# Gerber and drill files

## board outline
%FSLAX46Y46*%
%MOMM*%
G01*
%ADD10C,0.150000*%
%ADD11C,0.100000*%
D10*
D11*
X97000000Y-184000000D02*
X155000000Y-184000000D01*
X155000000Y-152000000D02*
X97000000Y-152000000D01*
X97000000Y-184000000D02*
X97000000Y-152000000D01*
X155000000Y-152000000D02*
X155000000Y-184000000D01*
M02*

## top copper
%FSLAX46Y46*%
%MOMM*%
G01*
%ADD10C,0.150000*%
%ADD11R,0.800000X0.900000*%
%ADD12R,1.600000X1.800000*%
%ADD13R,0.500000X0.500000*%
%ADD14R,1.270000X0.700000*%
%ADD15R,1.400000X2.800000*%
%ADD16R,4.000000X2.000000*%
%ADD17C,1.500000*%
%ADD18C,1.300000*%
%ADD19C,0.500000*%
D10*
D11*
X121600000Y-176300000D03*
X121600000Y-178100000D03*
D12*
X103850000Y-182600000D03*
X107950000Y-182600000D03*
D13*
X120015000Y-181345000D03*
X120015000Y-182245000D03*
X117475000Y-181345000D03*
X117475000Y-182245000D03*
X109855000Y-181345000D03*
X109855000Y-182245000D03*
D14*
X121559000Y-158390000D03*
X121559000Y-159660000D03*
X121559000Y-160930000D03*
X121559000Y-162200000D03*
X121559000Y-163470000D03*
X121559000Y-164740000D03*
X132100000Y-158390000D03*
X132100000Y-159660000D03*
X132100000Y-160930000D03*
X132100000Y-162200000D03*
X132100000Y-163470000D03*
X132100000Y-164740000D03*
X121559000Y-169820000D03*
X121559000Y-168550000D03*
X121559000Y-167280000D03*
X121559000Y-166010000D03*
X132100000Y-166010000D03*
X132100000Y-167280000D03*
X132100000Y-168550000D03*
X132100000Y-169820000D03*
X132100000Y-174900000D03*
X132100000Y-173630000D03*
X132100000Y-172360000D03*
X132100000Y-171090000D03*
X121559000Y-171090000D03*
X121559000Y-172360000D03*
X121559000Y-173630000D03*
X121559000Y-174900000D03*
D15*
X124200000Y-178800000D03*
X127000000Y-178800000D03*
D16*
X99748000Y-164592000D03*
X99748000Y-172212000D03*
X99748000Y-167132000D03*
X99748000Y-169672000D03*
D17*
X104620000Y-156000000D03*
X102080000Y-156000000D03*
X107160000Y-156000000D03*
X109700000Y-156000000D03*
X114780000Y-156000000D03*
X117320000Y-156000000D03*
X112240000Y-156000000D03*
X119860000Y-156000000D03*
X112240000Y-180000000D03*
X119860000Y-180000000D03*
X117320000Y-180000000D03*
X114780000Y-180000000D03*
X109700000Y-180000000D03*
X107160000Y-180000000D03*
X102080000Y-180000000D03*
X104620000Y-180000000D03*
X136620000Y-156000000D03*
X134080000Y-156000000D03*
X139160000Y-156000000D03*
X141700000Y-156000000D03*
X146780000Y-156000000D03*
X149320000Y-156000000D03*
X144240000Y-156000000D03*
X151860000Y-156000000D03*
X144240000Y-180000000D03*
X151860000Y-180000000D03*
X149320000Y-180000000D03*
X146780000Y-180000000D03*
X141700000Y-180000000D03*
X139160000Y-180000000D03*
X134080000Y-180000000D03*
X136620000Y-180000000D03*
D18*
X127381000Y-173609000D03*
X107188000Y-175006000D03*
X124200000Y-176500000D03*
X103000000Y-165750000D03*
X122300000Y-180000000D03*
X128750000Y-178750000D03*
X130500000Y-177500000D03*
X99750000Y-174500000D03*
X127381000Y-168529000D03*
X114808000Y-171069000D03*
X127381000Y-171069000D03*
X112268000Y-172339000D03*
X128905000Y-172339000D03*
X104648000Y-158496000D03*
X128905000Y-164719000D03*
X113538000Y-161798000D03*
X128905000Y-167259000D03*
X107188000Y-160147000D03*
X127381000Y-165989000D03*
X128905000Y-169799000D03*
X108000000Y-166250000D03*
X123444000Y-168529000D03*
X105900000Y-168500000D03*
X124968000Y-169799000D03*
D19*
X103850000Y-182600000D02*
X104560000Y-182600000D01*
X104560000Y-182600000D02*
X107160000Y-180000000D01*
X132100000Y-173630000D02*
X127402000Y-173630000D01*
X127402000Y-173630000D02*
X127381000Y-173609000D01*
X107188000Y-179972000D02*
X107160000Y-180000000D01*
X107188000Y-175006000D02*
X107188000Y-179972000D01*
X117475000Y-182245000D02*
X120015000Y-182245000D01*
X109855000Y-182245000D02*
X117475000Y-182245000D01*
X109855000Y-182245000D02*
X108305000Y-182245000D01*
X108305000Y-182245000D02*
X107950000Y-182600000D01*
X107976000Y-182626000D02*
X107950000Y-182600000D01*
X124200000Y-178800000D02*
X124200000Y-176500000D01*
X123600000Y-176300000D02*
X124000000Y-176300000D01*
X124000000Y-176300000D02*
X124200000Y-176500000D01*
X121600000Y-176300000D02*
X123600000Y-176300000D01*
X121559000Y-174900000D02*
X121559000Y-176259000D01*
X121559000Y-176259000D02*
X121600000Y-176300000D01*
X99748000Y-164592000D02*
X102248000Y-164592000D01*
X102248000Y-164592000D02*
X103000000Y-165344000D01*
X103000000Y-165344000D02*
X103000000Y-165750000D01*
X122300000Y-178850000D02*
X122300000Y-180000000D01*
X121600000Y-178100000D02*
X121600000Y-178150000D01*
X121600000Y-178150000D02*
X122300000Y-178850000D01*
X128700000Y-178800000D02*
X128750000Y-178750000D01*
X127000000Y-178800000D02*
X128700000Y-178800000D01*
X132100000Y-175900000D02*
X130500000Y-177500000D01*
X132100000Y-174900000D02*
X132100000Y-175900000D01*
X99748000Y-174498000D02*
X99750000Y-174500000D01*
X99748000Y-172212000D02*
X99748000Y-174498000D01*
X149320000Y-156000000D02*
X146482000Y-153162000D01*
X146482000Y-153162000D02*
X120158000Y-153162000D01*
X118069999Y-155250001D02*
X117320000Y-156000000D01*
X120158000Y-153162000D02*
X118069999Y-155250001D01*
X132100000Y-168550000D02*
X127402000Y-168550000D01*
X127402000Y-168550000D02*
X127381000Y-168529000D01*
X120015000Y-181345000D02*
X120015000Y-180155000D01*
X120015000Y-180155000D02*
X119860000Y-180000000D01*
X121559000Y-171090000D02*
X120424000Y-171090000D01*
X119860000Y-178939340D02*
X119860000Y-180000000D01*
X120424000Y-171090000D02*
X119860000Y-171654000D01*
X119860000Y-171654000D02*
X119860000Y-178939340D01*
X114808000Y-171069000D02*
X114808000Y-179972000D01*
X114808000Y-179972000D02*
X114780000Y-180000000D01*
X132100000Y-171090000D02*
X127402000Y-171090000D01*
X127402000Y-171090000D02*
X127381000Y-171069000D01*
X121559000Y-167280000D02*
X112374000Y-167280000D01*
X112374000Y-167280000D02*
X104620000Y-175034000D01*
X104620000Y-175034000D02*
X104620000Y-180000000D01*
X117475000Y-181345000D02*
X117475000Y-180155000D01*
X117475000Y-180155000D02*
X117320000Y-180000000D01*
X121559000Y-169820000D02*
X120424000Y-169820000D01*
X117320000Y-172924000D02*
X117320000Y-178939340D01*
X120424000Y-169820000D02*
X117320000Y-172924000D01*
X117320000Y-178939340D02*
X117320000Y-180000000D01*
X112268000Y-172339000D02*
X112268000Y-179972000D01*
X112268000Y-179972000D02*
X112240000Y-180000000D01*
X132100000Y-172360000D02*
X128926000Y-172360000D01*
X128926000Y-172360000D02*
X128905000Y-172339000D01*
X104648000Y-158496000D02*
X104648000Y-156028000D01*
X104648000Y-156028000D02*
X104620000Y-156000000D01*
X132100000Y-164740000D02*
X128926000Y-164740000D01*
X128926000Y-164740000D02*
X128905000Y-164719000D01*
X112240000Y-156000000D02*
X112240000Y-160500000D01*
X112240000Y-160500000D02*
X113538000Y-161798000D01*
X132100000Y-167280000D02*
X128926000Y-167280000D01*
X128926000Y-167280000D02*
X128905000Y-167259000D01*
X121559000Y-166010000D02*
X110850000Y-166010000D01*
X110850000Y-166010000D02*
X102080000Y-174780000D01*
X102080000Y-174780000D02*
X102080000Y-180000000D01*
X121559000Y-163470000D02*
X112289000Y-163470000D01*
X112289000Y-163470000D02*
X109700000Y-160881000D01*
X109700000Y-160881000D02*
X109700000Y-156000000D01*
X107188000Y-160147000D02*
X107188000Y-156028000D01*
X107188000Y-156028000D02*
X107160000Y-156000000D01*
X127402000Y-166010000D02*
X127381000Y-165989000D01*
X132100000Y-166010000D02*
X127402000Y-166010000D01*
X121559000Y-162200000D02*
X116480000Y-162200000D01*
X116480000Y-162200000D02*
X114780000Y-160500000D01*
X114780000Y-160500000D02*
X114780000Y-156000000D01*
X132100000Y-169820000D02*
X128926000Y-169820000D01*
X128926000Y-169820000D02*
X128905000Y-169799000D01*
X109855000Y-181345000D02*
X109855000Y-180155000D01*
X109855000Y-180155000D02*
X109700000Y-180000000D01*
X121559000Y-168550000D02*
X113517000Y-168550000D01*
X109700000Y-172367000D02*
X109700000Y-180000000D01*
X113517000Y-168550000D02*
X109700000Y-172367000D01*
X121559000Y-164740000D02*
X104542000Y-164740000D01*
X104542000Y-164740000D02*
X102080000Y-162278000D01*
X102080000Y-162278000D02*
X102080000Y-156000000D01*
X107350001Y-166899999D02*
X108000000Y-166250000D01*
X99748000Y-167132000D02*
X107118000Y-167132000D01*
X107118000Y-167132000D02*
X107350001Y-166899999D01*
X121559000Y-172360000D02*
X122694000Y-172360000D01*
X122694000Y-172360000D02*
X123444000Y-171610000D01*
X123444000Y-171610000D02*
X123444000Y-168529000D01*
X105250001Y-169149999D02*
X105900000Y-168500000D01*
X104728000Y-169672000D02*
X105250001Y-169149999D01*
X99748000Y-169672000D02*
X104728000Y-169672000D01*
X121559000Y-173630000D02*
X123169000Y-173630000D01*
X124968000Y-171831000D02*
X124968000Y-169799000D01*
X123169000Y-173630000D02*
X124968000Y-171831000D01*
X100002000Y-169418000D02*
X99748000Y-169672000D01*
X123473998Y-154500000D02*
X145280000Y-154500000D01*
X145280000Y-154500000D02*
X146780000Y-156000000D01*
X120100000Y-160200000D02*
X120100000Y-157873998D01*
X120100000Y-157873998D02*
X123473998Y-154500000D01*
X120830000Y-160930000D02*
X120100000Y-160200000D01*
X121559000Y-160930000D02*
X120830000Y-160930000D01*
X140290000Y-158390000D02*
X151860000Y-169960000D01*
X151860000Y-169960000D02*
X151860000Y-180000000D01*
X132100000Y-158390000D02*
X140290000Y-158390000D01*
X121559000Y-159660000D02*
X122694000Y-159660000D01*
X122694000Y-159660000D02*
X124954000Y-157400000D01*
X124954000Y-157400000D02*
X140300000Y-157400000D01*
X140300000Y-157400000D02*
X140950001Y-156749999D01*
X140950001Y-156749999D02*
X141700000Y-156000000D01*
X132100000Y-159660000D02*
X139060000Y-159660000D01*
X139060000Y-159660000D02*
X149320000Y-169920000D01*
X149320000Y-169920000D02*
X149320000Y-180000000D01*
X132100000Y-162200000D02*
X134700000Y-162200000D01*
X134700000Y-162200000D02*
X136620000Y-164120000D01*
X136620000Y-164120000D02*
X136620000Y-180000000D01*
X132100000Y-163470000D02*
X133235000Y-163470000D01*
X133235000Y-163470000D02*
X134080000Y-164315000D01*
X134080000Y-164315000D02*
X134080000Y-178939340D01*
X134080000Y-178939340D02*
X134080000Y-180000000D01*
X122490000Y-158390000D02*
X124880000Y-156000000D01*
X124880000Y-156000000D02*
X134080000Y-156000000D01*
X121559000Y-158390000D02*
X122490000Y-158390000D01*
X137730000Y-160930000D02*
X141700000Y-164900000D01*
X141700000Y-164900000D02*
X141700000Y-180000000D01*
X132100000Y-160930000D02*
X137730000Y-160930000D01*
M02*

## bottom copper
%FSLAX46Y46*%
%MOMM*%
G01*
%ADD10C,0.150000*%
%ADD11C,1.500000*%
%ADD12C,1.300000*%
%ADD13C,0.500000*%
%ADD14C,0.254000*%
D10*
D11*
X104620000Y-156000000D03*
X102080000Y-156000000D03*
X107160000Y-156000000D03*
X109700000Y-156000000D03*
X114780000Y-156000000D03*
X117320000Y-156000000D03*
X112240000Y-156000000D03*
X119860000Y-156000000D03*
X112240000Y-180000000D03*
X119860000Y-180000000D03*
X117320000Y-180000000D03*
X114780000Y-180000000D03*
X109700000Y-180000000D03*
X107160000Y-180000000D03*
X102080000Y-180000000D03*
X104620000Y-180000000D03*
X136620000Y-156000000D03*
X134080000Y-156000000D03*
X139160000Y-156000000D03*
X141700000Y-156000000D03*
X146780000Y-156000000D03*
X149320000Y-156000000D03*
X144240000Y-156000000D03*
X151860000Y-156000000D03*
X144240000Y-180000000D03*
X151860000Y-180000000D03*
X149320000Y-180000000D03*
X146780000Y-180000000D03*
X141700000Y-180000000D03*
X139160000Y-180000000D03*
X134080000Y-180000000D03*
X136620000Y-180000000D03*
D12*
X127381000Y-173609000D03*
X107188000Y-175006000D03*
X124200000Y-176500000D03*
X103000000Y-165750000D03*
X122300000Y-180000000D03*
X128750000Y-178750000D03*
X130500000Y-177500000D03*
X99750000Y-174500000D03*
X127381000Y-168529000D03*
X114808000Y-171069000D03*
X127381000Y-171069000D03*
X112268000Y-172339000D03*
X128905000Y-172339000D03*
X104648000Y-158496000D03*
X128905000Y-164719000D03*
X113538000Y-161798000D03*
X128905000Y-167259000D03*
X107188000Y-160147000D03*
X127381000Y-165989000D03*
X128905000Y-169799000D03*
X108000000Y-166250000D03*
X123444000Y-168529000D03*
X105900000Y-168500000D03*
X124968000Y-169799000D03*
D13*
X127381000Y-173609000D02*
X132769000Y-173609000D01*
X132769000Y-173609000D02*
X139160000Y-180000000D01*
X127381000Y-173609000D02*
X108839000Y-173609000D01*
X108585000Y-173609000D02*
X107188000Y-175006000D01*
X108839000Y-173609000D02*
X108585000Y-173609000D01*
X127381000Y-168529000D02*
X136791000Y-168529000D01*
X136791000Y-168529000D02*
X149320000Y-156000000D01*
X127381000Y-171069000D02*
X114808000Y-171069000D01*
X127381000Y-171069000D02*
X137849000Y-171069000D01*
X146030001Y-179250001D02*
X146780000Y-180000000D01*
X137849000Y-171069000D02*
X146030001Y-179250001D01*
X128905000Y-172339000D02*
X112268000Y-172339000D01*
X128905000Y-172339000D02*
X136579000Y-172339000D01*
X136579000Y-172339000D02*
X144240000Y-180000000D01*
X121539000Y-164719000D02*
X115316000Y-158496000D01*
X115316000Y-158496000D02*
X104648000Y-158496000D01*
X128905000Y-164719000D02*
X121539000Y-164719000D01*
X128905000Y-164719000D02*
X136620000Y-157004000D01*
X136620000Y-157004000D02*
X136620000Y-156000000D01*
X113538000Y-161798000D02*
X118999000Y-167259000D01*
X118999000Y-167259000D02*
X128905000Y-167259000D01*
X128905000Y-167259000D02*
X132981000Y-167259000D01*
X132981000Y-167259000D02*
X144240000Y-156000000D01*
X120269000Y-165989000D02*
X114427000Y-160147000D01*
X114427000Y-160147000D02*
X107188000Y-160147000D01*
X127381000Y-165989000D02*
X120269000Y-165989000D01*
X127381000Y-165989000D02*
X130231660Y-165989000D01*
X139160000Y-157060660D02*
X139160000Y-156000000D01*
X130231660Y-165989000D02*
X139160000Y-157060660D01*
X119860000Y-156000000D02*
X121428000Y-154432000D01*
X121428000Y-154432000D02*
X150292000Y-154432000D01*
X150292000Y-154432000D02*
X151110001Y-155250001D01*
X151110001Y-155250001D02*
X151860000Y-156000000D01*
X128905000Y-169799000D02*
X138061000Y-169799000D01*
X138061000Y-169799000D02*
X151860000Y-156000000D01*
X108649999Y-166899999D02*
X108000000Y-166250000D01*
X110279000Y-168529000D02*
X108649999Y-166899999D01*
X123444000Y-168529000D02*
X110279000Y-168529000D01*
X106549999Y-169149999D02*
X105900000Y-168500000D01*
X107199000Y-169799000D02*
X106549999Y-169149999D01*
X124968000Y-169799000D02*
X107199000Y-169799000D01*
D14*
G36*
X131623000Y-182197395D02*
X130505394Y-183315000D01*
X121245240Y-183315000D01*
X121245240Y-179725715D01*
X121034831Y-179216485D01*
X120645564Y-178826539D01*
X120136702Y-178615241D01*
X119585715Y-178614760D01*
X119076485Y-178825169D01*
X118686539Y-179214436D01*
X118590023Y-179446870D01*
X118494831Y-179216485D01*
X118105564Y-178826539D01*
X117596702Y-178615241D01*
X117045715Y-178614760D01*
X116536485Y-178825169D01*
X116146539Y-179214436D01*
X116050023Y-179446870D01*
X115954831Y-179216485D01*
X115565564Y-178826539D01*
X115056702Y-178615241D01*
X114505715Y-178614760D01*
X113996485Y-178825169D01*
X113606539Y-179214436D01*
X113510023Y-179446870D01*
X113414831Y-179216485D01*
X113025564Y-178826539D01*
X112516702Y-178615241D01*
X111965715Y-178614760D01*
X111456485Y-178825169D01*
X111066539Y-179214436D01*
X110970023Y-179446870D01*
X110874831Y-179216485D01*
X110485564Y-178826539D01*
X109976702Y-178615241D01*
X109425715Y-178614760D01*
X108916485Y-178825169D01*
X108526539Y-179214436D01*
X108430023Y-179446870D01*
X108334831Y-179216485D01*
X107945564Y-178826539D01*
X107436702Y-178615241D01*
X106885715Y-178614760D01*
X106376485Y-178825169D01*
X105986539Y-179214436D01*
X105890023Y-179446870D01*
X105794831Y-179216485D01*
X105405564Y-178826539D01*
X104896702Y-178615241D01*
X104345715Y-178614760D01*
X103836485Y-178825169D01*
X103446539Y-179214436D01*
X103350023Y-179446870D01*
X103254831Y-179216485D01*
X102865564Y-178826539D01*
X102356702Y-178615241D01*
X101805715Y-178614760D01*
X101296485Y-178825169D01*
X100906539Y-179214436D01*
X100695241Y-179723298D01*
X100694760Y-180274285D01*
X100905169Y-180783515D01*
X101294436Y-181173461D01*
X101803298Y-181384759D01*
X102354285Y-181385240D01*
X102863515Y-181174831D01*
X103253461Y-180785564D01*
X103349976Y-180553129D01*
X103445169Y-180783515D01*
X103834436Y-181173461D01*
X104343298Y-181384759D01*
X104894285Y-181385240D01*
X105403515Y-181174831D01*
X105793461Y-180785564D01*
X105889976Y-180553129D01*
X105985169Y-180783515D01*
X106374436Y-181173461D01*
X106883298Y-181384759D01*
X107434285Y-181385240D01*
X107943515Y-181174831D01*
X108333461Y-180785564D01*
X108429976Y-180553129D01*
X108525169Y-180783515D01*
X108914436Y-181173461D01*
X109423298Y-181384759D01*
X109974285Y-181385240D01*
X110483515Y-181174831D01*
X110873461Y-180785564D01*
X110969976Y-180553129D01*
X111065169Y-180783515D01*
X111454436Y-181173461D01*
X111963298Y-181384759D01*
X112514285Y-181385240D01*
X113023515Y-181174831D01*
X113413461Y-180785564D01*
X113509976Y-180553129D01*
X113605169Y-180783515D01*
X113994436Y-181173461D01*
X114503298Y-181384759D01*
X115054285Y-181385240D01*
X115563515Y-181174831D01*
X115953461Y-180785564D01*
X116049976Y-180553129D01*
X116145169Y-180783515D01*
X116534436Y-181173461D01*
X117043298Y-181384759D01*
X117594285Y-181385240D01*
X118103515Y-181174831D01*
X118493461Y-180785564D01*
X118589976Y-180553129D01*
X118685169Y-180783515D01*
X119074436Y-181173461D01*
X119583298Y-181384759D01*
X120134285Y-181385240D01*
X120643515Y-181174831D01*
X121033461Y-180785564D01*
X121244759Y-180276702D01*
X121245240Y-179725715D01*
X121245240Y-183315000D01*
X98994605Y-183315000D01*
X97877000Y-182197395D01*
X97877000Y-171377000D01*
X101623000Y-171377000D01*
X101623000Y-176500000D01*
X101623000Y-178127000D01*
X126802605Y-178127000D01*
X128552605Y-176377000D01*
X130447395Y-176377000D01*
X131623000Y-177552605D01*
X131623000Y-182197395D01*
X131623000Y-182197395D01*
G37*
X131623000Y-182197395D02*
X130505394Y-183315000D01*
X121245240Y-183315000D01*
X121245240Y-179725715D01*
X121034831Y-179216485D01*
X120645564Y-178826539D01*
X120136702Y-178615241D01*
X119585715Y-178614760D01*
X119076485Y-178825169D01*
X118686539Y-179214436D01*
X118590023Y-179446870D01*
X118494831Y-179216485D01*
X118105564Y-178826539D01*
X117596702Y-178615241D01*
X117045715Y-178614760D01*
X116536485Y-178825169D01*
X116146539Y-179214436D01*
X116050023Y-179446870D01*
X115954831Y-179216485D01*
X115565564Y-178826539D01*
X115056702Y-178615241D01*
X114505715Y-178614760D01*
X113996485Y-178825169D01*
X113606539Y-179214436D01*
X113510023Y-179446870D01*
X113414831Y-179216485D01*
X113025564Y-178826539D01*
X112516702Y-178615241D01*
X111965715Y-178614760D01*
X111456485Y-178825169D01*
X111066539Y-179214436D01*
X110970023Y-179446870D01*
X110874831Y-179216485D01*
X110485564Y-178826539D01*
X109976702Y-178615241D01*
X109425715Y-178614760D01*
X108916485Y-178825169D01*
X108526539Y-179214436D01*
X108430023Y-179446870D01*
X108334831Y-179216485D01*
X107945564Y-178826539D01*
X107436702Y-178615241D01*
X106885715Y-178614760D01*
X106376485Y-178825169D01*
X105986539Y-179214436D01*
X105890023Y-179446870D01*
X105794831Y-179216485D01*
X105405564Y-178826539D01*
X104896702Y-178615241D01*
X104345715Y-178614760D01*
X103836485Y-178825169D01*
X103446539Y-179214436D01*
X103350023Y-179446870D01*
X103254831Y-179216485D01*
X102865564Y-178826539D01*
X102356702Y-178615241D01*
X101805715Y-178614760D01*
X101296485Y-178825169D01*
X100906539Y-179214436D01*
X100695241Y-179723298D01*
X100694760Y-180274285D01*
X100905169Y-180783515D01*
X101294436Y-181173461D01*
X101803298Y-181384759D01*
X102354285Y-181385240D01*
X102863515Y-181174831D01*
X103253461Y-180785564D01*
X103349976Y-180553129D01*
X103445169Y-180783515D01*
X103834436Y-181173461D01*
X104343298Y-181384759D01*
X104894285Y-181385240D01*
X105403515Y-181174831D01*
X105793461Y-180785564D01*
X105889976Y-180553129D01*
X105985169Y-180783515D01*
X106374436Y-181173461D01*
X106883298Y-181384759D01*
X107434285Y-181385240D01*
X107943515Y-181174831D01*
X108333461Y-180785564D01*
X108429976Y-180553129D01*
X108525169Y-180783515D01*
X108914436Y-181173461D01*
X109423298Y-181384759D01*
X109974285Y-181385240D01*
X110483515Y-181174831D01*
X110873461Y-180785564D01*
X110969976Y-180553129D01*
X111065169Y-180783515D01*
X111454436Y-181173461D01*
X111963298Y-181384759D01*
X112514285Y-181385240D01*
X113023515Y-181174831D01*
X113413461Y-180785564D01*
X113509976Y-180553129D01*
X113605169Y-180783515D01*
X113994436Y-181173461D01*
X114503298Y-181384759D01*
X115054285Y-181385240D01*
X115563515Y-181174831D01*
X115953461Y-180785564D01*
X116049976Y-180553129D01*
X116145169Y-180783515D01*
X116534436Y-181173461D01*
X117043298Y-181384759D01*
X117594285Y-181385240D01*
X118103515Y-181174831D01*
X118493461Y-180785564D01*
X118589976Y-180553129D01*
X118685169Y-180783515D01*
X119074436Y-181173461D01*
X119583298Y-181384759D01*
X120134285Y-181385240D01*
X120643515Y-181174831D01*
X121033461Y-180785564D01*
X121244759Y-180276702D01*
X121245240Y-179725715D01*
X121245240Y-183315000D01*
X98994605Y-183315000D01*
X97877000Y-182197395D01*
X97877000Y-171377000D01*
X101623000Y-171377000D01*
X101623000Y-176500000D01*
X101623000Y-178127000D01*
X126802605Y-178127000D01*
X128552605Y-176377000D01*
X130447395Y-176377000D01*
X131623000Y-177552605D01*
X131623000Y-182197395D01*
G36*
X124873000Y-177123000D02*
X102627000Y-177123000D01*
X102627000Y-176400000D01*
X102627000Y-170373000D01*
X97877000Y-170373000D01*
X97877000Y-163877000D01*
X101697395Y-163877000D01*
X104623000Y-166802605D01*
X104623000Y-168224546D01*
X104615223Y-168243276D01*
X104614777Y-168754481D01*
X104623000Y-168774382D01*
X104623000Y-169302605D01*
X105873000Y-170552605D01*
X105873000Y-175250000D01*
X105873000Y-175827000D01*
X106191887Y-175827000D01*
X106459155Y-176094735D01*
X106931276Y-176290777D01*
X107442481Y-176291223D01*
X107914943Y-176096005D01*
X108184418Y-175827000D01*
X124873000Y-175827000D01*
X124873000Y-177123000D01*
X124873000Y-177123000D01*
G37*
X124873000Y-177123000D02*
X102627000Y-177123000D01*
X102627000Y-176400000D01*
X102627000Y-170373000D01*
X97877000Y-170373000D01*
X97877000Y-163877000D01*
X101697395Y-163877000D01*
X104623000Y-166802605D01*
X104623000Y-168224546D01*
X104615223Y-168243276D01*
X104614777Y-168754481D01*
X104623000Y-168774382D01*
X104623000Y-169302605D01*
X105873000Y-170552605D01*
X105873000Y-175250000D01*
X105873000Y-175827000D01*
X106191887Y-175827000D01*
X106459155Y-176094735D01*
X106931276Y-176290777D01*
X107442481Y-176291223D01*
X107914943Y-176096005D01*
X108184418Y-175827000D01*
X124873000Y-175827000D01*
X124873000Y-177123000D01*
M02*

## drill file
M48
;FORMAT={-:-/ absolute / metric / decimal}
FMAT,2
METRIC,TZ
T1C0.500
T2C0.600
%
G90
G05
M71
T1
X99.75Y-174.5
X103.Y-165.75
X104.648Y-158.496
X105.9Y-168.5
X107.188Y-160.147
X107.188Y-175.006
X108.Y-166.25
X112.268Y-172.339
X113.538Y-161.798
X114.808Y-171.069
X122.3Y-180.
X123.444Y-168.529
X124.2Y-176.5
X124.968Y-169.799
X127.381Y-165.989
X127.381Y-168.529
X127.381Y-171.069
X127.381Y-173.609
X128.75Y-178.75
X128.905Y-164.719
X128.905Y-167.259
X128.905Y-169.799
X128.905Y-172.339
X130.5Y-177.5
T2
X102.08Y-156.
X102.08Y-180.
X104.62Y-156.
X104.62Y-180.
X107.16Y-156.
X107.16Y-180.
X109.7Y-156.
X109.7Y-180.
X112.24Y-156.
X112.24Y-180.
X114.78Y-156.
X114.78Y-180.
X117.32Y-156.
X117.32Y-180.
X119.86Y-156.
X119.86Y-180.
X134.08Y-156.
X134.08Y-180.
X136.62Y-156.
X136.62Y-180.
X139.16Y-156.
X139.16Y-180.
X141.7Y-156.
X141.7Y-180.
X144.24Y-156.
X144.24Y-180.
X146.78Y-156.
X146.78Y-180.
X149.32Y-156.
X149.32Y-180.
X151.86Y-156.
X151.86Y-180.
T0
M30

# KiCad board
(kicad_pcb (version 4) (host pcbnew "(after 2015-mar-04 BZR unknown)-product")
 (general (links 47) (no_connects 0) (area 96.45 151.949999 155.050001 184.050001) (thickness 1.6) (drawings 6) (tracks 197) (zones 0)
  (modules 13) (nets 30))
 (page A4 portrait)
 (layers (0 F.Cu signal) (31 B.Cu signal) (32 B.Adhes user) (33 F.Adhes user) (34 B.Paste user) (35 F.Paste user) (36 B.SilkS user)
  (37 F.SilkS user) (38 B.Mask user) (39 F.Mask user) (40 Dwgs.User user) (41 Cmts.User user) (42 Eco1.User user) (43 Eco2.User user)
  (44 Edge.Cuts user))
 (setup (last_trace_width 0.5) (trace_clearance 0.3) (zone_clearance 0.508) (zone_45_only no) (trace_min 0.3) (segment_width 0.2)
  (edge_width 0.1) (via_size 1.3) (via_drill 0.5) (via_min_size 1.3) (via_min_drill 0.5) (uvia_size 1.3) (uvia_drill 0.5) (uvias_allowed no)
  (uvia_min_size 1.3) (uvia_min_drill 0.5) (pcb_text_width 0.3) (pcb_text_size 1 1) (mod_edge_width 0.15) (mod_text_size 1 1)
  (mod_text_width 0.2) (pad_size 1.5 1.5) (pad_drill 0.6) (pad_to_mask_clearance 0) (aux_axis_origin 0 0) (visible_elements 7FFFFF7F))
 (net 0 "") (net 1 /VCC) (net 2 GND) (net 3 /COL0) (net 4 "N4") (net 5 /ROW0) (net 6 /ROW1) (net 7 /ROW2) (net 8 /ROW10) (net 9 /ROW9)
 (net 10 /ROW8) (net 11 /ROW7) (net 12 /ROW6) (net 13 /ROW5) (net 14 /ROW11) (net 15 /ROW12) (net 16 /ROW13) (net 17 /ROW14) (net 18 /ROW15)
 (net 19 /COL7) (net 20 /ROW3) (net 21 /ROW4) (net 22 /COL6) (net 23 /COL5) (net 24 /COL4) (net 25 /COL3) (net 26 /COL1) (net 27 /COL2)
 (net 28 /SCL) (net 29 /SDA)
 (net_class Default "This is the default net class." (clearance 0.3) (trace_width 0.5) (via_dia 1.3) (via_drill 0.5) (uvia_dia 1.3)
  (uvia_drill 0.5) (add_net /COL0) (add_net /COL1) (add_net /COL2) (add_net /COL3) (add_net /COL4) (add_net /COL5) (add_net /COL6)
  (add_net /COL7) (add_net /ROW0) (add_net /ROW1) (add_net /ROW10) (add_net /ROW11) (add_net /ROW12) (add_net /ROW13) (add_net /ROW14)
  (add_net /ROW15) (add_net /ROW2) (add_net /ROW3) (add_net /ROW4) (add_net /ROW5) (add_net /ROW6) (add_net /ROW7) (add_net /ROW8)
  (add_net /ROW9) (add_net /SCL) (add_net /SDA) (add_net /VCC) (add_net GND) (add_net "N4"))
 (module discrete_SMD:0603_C (layer F.Cu) (at 121.6 176.45 270)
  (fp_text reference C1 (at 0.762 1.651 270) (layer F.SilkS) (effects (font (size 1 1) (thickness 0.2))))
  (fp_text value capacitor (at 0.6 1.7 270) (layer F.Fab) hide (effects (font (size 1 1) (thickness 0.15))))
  (pad 1 smd rect (at -0.15 0 270) (size 0.9 0.8) (layers F.Cu F.Paste F.Mask) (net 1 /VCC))
  (pad 2 smd rect (at 1.65 0 270) (size 0.9 0.8) (layers F.Cu F.Paste F.Mask) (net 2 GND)))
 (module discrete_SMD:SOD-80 (layer F.Cu) (at 104.25 182.6 270)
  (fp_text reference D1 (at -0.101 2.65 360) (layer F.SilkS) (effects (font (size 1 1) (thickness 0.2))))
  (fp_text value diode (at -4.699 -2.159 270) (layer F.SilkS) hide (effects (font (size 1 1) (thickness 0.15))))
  (pad 1 smd rect (at 0 0.4 270) (size 1.8 1.6) (layers F.Cu F.Paste F.Mask) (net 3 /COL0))
  (pad 2 smd rect (at 0 -3.7 270) (size 1.8 1.6) (layers F.Cu F.Paste F.Mask) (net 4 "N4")))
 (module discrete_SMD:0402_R (layer F.Cu) (at 120.015 181.345 270)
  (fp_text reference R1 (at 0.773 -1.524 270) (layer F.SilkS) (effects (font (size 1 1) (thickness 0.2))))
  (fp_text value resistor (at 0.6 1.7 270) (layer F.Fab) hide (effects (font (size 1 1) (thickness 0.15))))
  (pad 1 smd rect (at 0 0 270) (size 0.5 0.5) (layers F.Cu F.Paste F.Mask) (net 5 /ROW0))
  (pad 2 smd rect (at 0.9 0 270) (size 0.5 0.5) (layers F.Cu F.Paste F.Mask) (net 4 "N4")))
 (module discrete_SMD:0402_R (layer F.Cu) (at 117.475 181.345 270)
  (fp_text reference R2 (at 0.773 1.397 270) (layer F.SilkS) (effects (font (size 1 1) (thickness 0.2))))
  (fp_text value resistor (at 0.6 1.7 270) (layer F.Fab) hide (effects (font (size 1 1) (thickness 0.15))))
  (pad 1 smd rect (at 0 0 270) (size 0.5 0.5) (layers F.Cu F.Paste F.Mask) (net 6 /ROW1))
  (pad 2 smd rect (at 0.9 0 270) (size 0.5 0.5) (layers F.Cu F.Paste F.Mask) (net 4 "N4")))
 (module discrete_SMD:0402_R (layer F.Cu) (at 109.855 181.345 270)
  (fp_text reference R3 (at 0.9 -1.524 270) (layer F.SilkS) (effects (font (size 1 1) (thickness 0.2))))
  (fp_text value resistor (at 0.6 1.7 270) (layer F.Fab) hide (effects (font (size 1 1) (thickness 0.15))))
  (pad 1 smd rect (at 0 0 270) (size 0.5 0.5) (layers F.Cu F.Paste F.Mask) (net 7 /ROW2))
  (pad 2 smd rect (at 0.9 0 270) (size 0.5 0.5) (layers F.Cu F.Paste F.Mask) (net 4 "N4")))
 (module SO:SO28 (layer F.Cu) (at 132.1 174.9 90)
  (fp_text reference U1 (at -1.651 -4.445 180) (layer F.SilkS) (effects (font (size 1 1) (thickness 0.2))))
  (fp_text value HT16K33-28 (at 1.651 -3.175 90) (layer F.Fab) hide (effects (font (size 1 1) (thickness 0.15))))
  (pad 15 smd rect (at 16.51 -10.541 90) (size 0.7 1.27) (layers F.Cu F.Paste F.Mask) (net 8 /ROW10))
  (pad 16 smd rect (at 15.24 -10.541 90) (size 0.7 1.27) (layers F.Cu F.Paste F.Mask) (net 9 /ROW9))
  (pad 17 smd rect (at 13.97 -10.541 90) (size 0.7 1.27) (layers F.Cu F.Paste F.Mask) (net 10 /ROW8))
  (pad 18 smd rect (at 12.7 -10.541 90) (size 0.7 1.27) (layers F.Cu F.Paste F.Mask) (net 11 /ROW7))
  (pad 19 smd rect (at 11.43 -10.541 90) (size 0.7 1.27) (layers F.Cu F.Paste F.Mask) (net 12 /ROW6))
  (pad 20 smd rect (at 10.16 -10.541 90) (size 0.7 1.27) (layers F.Cu F.Paste F.Mask) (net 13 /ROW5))
  (pad 14 smd rect (at 16.51 0 90) (size 0.7 1.27) (layers F.Cu F.Paste F.Mask) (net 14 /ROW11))
  (pad 13 smd rect (at 15.24 0 90) (size 0.7 1.27) (layers F.Cu F.Paste F.Mask) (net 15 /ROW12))
  (pad 12 smd rect (at 13.97 0 90) (size 0.7 1.27) (layers F.Cu F.Paste F.Mask) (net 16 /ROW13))
  (pad 11 smd rect (at 12.7 0 90) (size 0.7 1.27) (layers F.Cu F.Paste F.Mask) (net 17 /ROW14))
  (pad 10 smd rect (at 11.43 0 90) (size 0.7 1.27) (layers F.Cu F.Paste F.Mask) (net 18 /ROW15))
  (pad 9 smd rect (at 10.16 0 90) (size 0.7 1.27) (layers F.Cu F.Paste F.Mask) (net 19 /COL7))
  (pad 24 smd rect (at 5.08 -10.541 90) (size 0.7 1.27) (layers F.Cu F.Paste F.Mask) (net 6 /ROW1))
  (pad 23 smd rect (at 6.35 -10.541 90) (size 0.7 1.27) (layers F.Cu F.Paste F.Mask) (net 7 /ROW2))
  (pad 22 smd rect (at 7.62 -10.541 90) (size 0.7 1.27) (layers F.Cu F.Paste F.Mask) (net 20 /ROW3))
  (pad 21 smd rect (at 8.89 -10.541 90) (size 0.7 1.27) (layers F.Cu F.Paste F.Mask) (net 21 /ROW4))
  (pad 8 smd rect (at 8.89 0 90) (size 0.7 1.27) (layers F.Cu F.Paste F.Mask) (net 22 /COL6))
  (pad 7 smd rect (at 7.62 0 90) (size 0.7 1.27) (layers F.Cu F.Paste F.Mask) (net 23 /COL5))
  (pad 6 smd rect (at 6.35 0 90) (size 0.7 1.27) (layers F.Cu F.Paste F.Mask) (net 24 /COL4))
  (pad 5 smd rect (at 5.08 0 90) (size 0.7 1.27) (layers F.Cu F.Paste F.Mask) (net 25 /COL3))
  (pad 1 smd rect (at 0 0 90) (size 0.7 1.27) (layers F.Cu F.Paste F.Mask) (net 2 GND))
  (pad 2 smd rect (at 1.27 0 90) (size 0.7 1.27) (layers F.Cu F.Paste F.Mask) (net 3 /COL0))
  (pad 3 smd rect (at 2.54 0 90) (size 0.7 1.27) (layers F.Cu F.Paste F.Mask) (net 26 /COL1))
  (pad 4 smd rect (at 3.81 0 90) (size 0.7 1.27) (layers F.Cu F.Paste F.Mask) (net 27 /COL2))
  (pad 25 smd rect (at 3.81 -10.541 90) (size 0.7 1.27) (layers F.Cu F.Paste F.Mask) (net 5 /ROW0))
  (pad 26 smd rect (at 2.54 -10.541 90) (size 0.7 1.27) (layers F.Cu F.Paste F.Mask) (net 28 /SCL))
  (pad 27 smd rect (at 1.27 -10.541 90) (size 0.7 1.27) (layers F.Cu F.Paste F.Mask) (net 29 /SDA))
  (pad 28 smd rect (at 0 -10.541 90) (size 0.7 1.27) (layers F.Cu F.Paste F.Mask) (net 1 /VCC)))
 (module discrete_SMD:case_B (layer F.Cu) (at 125.65 178.8)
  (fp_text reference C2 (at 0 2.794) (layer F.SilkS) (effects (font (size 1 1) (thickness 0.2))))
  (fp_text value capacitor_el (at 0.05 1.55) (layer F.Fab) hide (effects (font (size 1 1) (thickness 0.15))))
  (pad 1 smd rect (at -1.45 0) (size 1.4 2.8) (layers F.Cu F.Paste F.Mask) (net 1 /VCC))
  (pad 2 smd rect (at 1.35 0) (size 1.4 2.8) (layers F.Cu F.Paste F.Mask) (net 2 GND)))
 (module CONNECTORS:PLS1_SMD (layer F.Cu) (at 98.298 164.592)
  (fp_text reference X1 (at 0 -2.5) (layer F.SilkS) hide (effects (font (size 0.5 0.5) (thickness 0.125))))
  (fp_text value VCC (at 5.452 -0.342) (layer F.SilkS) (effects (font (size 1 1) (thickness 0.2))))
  (pad 1 smd rect (at 1.45 0) (size 4 2) (layers F.Cu F.Paste F.Mask) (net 1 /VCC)))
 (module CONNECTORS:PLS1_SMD (layer F.Cu) (at 98.298 172.212)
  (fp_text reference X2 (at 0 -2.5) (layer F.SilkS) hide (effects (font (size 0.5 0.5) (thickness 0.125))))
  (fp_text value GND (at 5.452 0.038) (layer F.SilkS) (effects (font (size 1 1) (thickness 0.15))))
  (pad 1 smd rect (at 1.45 0) (size 4 2) (layers F.Cu F.Paste F.Mask) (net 2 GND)))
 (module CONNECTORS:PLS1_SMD (layer F.Cu) (at 98.298 167.132)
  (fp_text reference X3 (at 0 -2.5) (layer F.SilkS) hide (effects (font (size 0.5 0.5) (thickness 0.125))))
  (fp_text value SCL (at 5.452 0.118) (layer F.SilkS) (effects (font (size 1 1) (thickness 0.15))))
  (pad 1 smd rect (at 1.45 0) (size 4 2) (layers F.Cu F.Paste F.Mask) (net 28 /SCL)))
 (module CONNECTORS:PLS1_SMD (layer F.Cu) (at 98.298 169.672)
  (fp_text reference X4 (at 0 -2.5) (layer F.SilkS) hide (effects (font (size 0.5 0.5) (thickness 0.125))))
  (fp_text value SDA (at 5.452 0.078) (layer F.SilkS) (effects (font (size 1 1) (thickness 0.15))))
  (pad 1 smd rect (at 1.45 0) (size 4 2) (layers F.Cu F.Paste F.Mask) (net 29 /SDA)))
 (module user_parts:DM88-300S (layer B.Cu) (at 97 156)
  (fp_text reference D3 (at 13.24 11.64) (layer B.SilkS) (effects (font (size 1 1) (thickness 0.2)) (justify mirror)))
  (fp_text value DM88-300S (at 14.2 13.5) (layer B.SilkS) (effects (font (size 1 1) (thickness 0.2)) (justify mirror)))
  (pad 2 thru_hole circle (at 7.62 0) (size 1.5 1.5) (drill 0.6) (layers *.Cu *.Mask) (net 19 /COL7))
  (pad 1 thru_hole circle (at 5.08 0) (size 1.5 1.5) (drill 0.6) (layers *.Cu *.Mask) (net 13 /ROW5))
  (pad 3 thru_hole circle (at 10.16 0) (size 1.5 1.5) (drill 0.6) (layers *.Cu *.Mask) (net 22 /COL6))
  (pad 4 thru_hole circle (at 12.7 0) (size 1.5 1.5) (drill 0.6) (layers *.Cu *.Mask) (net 12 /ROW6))
  (pad 6 thru_hole circle (at 17.78 0) (size 1.5 1.5) (drill 0.6) (layers *.Cu *.Mask) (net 11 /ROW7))
  (pad 7 thru_hole circle (at 20.32 0) (size 1.5 1.5) (drill 0.6) (layers *.Cu *.Mask) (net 24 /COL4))
  (pad 5 thru_hole circle (at 15.24 0) (size 1.5 1.5) (drill 0.6) (layers *.Cu *.Mask) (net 23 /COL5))
  (pad 8 thru_hole circle (at 22.86 0) (size 1.5 1.5) (drill 0.6) (layers *.Cu *.Mask) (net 25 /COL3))
  (pad 12 thru_hole circle (at 15.24 24) (size 1.5 1.5) (drill 0.6) (layers *.Cu *.Mask) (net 26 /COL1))
  (pad 9 thru_hole circle (at 22.86 24) (size 1.5 1.5) (drill 0.6) (layers *.Cu *.Mask) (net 5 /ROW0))
  (pad 10 thru_hole circle (at 20.32 24) (size 1.5 1.5) (drill 0.6) (layers *.Cu *.Mask) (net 6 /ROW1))
  (pad 11 thru_hole circle (at 17.78 24) (size 1.5 1.5) (drill 0.6) (layers *.Cu *.Mask) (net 27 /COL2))
  (pad 13 thru_hole circle (at 12.7 24) (size 1.5 1.5) (drill 0.6) (layers *.Cu *.Mask) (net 7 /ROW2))
  (pad 14 thru_hole circle (at 10.16 24) (size 1.5 1.5) (drill 0.6) (layers *.Cu *.Mask) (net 3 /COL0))
  (pad 16 thru_hole circle (at 5.08 24) (size 1.5 1.5) (drill 0.6) (layers *.Cu *.Mask) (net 21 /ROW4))
  (pad 15 thru_hole circle (at 7.62 24) (size 1.5 1.5) (drill 0.6) (layers *.Cu *.Mask) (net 20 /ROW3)))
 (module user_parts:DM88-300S (layer B.Cu) (at 129 156)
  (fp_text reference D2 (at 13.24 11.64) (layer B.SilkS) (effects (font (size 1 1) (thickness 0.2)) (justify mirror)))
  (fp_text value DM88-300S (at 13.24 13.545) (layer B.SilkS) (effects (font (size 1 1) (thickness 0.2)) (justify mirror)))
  (pad 2 thru_hole circle (at 7.62 0) (size 1.5 1.5) (drill 0.6) (layers *.Cu *.Mask) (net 19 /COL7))
  (pad 1 thru_hole circle (at 5.08 0) (size 1.5 1.5) (drill 0.6) (layers *.Cu *.Mask) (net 8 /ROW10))
  (pad 3 thru_hole circle (at 10.16 0) (size 1.5 1.5) (drill 0.6) (layers *.Cu *.Mask) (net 22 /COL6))
  (pad 4 thru_hole circle (at 12.7 0) (size 1.5 1.5) (drill 0.6) (layers *.Cu *.Mask) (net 9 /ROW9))
  (pad 6 thru_hole circle (at 17.78 0) (size 1.5 1.5) (drill 0.6) (layers *.Cu *.Mask) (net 10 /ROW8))
  (pad 7 thru_hole circle (at 20.32 0) (size 1.5 1.5) (drill 0.6) (layers *.Cu *.Mask) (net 24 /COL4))
  (pad 5 thru_hole circle (at 15.24 0) (size 1.5 1.5) (drill 0.6) (layers *.Cu *.Mask) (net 23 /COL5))
  (pad 8 thru_hole circle (at 22.86 0) (size 1.5 1.5) (drill 0.6) (layers *.Cu *.Mask) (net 25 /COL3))
  (pad 12 thru_hole circle (at 15.24 24) (size 1.5 1.5) (drill 0.6) (layers *.Cu *.Mask) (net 26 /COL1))
  (pad 9 thru_hole circle (at 22.86 24) (size 1.5 1.5) (drill 0.6) (layers *.Cu *.Mask) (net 14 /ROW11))
  (pad 10 thru_hole circle (at 20.32 24) (size 1.5 1.5) (drill 0.6) (layers *.Cu *.Mask) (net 15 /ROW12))
  (pad 11 thru_hole circle (at 17.78 24) (size 1.5 1.5) (drill 0.6) (layers *.Cu *.Mask) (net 27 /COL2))
  (pad 13 thru_hole circle (at 12.7 24) (size 1.5 1.5) (drill 0.6) (layers *.Cu *.Mask) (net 16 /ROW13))
  (pad 14 thru_hole circle (at 10.16 24) (size 1.5 1.5) (drill 0.6) (layers *.Cu *.Mask) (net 3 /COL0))
  (pad 16 thru_hole circle (at 5.08 24) (size 1.5 1.5) (drill 0.6) (layers *.Cu *.Mask) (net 18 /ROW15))
  (pad 15 thru_hole circle (at 7.62 24) (size 1.5 1.5) (drill 0.6) (layers *.Cu *.Mask) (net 17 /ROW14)))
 (gr_line (start 97 184) (end 155 184) (angle 90) (layer Edge.Cuts) (width 0.1))
 (gr_line (start 155 152) (end 97 152) (angle 90) (layer Edge.Cuts) (width 0.1))
 (gr_line (start 97 184) (end 97 152) (angle 90) (layer Edge.Cuts) (width 0.1))
 (gr_line (start 155 152) (end 155 184) (angle 90) (layer Edge.Cuts) (width 0.1))
 (segment (start 103.85 182.6) (end 104.56 182.6) (width 0.5) (layer F.Cu) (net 3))
 (segment (start 104.56 182.6) (end 107.16 180) (width 0.5) (layer F.Cu) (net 3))
 (segment (start 127.381 173.609) (end 132.769 173.609) (width 0.5) (layer B.Cu) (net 3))
 (segment (start 132.769 173.609) (end 139.16 180) (width 0.5) (layer B.Cu) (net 3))
 (segment (start 132.1 173.63) (end 127.402 173.63) (width 0.5) (layer F.Cu) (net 3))
 (via (at 127.381 173.609) (size 1.3) (drill 0.5) (layers F.Cu B.Cu) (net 3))
 (segment (start 127.402 173.63) (end 127.381 173.609) (width 0.5) (layer F.Cu) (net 3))
 (segment (start 127.381 173.609) (end 108.839 173.609) (width 0.5) (layer B.Cu) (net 3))
 (via (at 107.188 175.006) (size 1.3) (drill 0.5) (layers F.Cu B.Cu) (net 3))
 (segment (start 108.585 173.609) (end 107.188 175.006) (width 0.5) (layer B.Cu) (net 3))
 (segment (start 108.839 173.609) (end 108.585 173.609) (width 0.5) (layer B.Cu) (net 3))
 (segment (start 107.188 179.972) (end 107.16 180) (width 0.5) (layer F.Cu) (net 3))
 (segment (start 107.188 175.006) (end 107.188 179.972) (width 0.5) (layer F.Cu) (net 3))
 (segment (start 109.855 182.245) (end 117.475 182.245) (width 0.5) (layer F.Cu) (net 4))
 (segment (start 117.475 182.245) (end 120.015 182.245) (width 0.5) (layer F.Cu) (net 4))
 (segment (start 109.855 182.245) (end 108.305 182.245) (width 0.5) (layer F.Cu) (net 4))
 (segment (start 108.305 182.245) (end 107.95 182.6) (width 0.5) (layer F.Cu) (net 4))
 (segment (start 107.976 182.626) (end 107.95 182.6) (width 0.5) (layer F.Cu) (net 4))
 (segment (start 124.2 178.8) (end 124.2 176.5) (width 0.5) (layer F.Cu) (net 1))
 (segment (start 123.6 176.3) (end 124 176.3) (width 0.5) (layer F.Cu) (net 1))
 (segment (start 124 176.3) (end 124.2 176.5) (width 0.5) (layer F.Cu) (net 1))
 (via (at 124.2 176.5) (size 1.3) (drill 0.5) (layers F.Cu B.Cu) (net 1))
 (segment (start 121.6 176.3) (end 123.6 176.3) (width 0.5) (layer F.Cu) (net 1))
 (segment (start 121.559 174.9) (end 121.559 176.259) (width 0.5) (layer F.Cu) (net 1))
 (segment (start 121.559 176.259) (end 121.6 176.3) (width 0.5) (layer F.Cu) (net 1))
 (via (at 103 165.75) (size 1.3) (drill 0.5) (layers F.Cu B.Cu) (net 1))
 (segment (start 99.748 164.592) (end 102.248 164.592) (width 0.5) (layer F.Cu) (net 1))
 (segment (start 102.248 164.592) (end 103 165.344) (width 0.5) (layer F.Cu) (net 1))
 (segment (start 103 165.344) (end 103 165.75) (width 0.5) (layer F.Cu) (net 1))
 (segment (start 122.3 178.85) (end 122.3 180) (width 0.5) (layer F.Cu) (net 2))
 (via (at 122.3 180) (size 1.3) (drill 0.5) (layers F.Cu B.Cu) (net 2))
 (segment (start 121.6 178.1) (end 121.6 178.15) (width 0.5) (layer F.Cu) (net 2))
 (segment (start 121.6 178.15) (end 122.3 178.85) (width 0.5) (layer F.Cu) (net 2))
 (via (at 128.75 178.75) (size 1.3) (drill 0.5) (layers F.Cu B.Cu) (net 2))
 (segment (start 128.7 178.8) (end 128.75 178.75) (width 0.5) (layer F.Cu) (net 2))
 (segment (start 127 178.8) (end 128.7 178.8) (width 0.5) (layer F.Cu) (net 2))
 (via (at 130.5 177.5) (size 1.3) (drill 0.5) (layers F.Cu B.Cu) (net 2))
 (segment (start 132.1 175.9) (end 130.5 177.5) (width 0.5) (layer F.Cu) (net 2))
 (segment (start 132.1 174.9) (end 132.1 175.9) (width 0.5) (layer F.Cu) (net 2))
 (via (at 99.75 174.5) (size 1.3) (drill 0.5) (layers F.Cu B.Cu) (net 2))
 (segment (start 99.748 174.498) (end 99.75 174.5) (width 0.5) (layer F.Cu) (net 2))
 (segment (start 99.748 172.212) (end 99.748 174.498) (width 0.5) (layer F.Cu) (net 2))
 (segment (start 149.32 156) (end 146.482 153.162) (width 0.5) (layer F.Cu) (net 24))
 (segment (start 146.482 153.162) (end 120.158 153.162) (width 0.5) (layer F.Cu) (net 24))
 (segment (start 118.069999 155.250001) (end 117.32 156) (width 0.5) (layer F.Cu) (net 24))
 (segment (start 120.158 153.162) (end 118.069999 155.250001) (width 0.5) (layer F.Cu) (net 24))
 (segment (start 127.381 168.529) (end 136.791 168.529) (width 0.5) (layer B.Cu) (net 24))
 (segment (start 136.791 168.529) (end 149.32 156) (width 0.5) (layer B.Cu) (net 24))
 (segment (start 132.1 168.55) (end 127.402 168.55) (width 0.5) (layer F.Cu) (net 24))
 (segment (start 127.402 168.55) (end 127.381 168.529) (width 0.5) (layer F.Cu) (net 24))
 (via (at 127.381 168.529) (size 1.3) (drill 0.5) (layers F.Cu B.Cu) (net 24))
 (segment (start 120.015 181.345) (end 120.015 180.155) (width 0.5) (layer F.Cu) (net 5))
 (segment (start 120.015 180.155) (end 119.86 180) (width 0.5) (layer F.Cu) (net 5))
 (segment (start 121.559 171.09) (end 120.424 171.09) (width 0.5) (layer F.Cu) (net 5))
 (segment (start 119.86 178.93934) (end 119.86 180) (width 0.5) (layer F.Cu) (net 5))
 (segment (start 120.424 171.09) (end 119.86 171.654) (width 0.5) (layer F.Cu) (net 5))
 (segment (start 119.86 171.654) (end 119.86 178.93934) (width 0.5) (layer F.Cu) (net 5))
 (segment (start 114.808 171.069) (end 114.808 179.972) (width 0.5) (layer F.Cu) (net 27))
 (segment (start 114.808 179.972) (end 114.78 180) (width 0.5) (layer F.Cu) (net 27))
 (segment (start 127.381 171.069) (end 114.808 171.069) (width 0.5) (layer B.Cu) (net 27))
 (via (at 114.808 171.069) (size 1.3) (drill 0.5) (layers F.Cu B.Cu) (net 27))
 (segment (start 127.381 171.069) (end 137.849 171.069) (width 0.5) (layer B.Cu) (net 27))
 (segment (start 146.030001 179.250001) (end 146.78 180) (width 0.5) (layer B.Cu) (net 27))
 (segment (start 137.849 171.069) (end 146.030001 179.250001) (width 0.5) (layer B.Cu) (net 27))
 (segment (start 132.1 171.09) (end 127.402 171.09) (width 0.5) (layer F.Cu) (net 27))
 (segment (start 127.402 171.09) (end 127.381 171.069) (width 0.5) (layer F.Cu) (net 27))
 (via (at 127.381 171.069) (size 1.3) (drill 0.5) (layers F.Cu B.Cu) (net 27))
 (segment (start 121.559 167.28) (end 112.374 167.28) (width 0.5) (layer F.Cu) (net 20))
 (segment (start 112.374 167.28) (end 104.62 175.034) (width 0.5) (layer F.Cu) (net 20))
 (segment (start 104.62 175.034) (end 104.62 180) (width 0.5) (layer F.Cu) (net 20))
 (segment (start 117.475 181.345) (end 117.475 180.155) (width 0.5) (layer F.Cu) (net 6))
 (segment (start 117.475 180.155) (end 117.32 180) (width 0.5) (layer F.Cu) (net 6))
 (segment (start 121.559 169.82) (end 120.424 169.82) (width 0.5) (layer F.Cu) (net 6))
 (segment (start 117.32 172.924) (end 117.32 178.93934) (width 0.5) (layer F.Cu) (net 6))
 (segment (start 120.424 169.82) (end 117.32 172.924) (width 0.5) (layer F.Cu) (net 6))
 (segment (start 117.32 178.93934) (end 117.32 180) (width 0.5) (layer F.Cu) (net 6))
 (segment (start 112.268 172.339) (end 112.268 179.972) (width 0.5) (layer F.Cu) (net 26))
 (segment (start 112.268 179.972) (end 112.24 180) (width 0.5) (layer F.Cu) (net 26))
 (segment (start 128.905 172.339) (end 112.268 172.339) (width 0.5) (layer B.Cu) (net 26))
 (via (at 112.268 172.339) (size 1.3) (drill 0.5) (layers F.Cu B.Cu) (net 26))
 (segment (start 128.905 172.339) (end 136.579 172.339) (width 0.5) (layer B.Cu) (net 26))
 (segment (start 136.579 172.339) (end 144.24 180) (width 0.5) (layer B.Cu) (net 26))
 (segment (start 132.1 172.36) (end 128.926 172.36) (width 0.5) (layer F.Cu) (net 26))
 (segment (start 128.926 172.36) (end 128.905 172.339) (width 0.5) (layer F.Cu) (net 26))
 (via (at 128.905 172.339) (size 1.3) (drill 0.5) (layers F.Cu B.Cu) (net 26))
 (segment (start 104.648 158.496) (end 104.648 156.028) (width 0.5) (layer F.Cu) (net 19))
 (segment (start 104.648 156.028) (end 104.62 156) (width 0.5) (layer F.Cu) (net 19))
 (segment (start 121.539 164.719) (end 115.316 158.496) (width 0.5) (layer B.Cu) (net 19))
 (segment (start 115.316 158.496) (end 104.648 158.496) (width 0.5) (layer B.Cu) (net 19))
 (via (at 104.648 158.496) (size 1.3) (drill 0.5) (layers F.Cu B.Cu) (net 19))
 (segment (start 128.905 164.719) (end 121.539 164.719) (width 0.5) (layer B.Cu) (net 19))
 (segment (start 128.905 164.719) (end 136.62 157.004) (width 0.5) (layer B.Cu) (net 19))
 (via (at 128.905 164.719) (size 1.3) (drill 0.5) (layers F.Cu B.Cu) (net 19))
 (segment (start 132.1 164.74) (end 128.926 164.74) (width 0.5) (layer F.Cu) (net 19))
 (segment (start 128.926 164.74) (end 128.905 164.719) (width 0.5) (layer F.Cu) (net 19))
 (segment (start 136.62 157.004) (end 136.62 156) (width 0.5) (layer B.Cu) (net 19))
 (segment (start 113.538 161.798) (end 118.999 167.259) (width 0.5) (layer B.Cu) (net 23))
 (segment (start 118.999 167.259) (end 128.905 167.259) (width 0.5) (layer B.Cu) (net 23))
 (segment (start 112.24 156) (end 112.24 160.5) (width 0.5) (layer F.Cu) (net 23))
 (segment (start 112.24 160.5) (end 113.538 161.798) (width 0.5) (layer F.Cu) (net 23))
 (via (at 113.538 161.798) (size 1.3) (drill 0.5) (layers F.Cu B.Cu) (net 23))
 (segment (start 128.905 167.259) (end 132.981 167.259) (width 0.5) (layer B.Cu) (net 23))
 (segment (start 132.981 167.259) (end 144.24 156) (width 0.5) (layer B.Cu) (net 23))
 (segment (start 132.1 167.28) (end 128.926 167.28) (width 0.5) (layer F.Cu) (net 23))
 (segment (start 128.926 167.28) (end 128.905 167.259) (width 0.5) (layer F.Cu) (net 23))
 (via (at 128.905 167.259) (size 1.3) (drill 0.5) (layers F.Cu B.Cu) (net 23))
 (segment (start 121.559 166.01) (end 110.85 166.01) (width 0.5) (layer F.Cu) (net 21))
 (segment (start 110.85 166.01) (end 102.08 174.78) (width 0.5) (layer F.Cu) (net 21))
 (segment (start 102.08 174.78) (end 102.08 180) (width 0.5) (layer F.Cu) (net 21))
 (segment (start 121.559 163.47) (end 112.289 163.47) (width 0.5) (layer F.Cu) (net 12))
 (segment (start 112.289 163.47) (end 109.7 160.881) (width 0.5) (layer F.Cu) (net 12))
 (segment (start 109.7 160.881) (end 109.7 156) (width 0.5) (layer F.Cu) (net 12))
 (segment (start 107.188 160.147) (end 107.188 156.028) (width 0.5) (layer F.Cu) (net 22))
 (segment (start 107.188 156.028) (end 107.16 156) (width 0.5) (layer F.Cu) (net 22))
 (segment (start 120.269 165.989) (end 114.427 160.147) (width 0.5) (layer B.Cu) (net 22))
 (via (at 107.188 160.147) (size 1.3) (drill 0.5) (layers F.Cu B.Cu) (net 22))
 (segment (start 114.427 160.147) (end 107.188 160.147) (width 0.5) (layer B.Cu) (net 22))
 (segment (start 127.381 165.989) (end 120.269 165.989) (width 0.5) (layer B.Cu) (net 22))
 (segment (start 127.402 166.01) (end 127.381 165.989) (width 0.5) (layer F.Cu) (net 22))
 (segment (start 132.1 166.01) (end 127.402 166.01) (width 0.5) (layer F.Cu) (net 22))
 (segment (start 127.381 165.989) (end 130.23166 165.989) (width 0.5) (layer B.Cu) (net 22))
 (via (at 127.381 165.989) (size 1.3) (drill 0.5) (layers F.Cu B.Cu) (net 22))
 (segment (start 139.16 157.06066) (end 139.16 156) (width 0.5) (layer B.Cu) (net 22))
 (segment (start 130.23166 165.989) (end 139.16 157.06066) (width 0.5) (layer B.Cu) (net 22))
 (segment (start 121.559 162.2) (end 116.48 162.2) (width 0.5) (layer F.Cu) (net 11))
 (segment (start 116.48 162.2) (end 114.78 160.5) (width 0.5) (layer F.Cu) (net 11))
 (segment (start 114.78 160.5) (end 114.78 156) (width 0.5) (layer F.Cu) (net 11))
 (segment (start 119.86 156) (end 121.428 154.432) (width 0.5) (layer B.Cu) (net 25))
 (segment (start 121.428 154.432) (end 150.292 154.432) (width 0.5) (layer B.Cu) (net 25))
 (segment (start 150.292 154.432) (end 151.110001 155.250001) (width 0.5) (layer B.Cu) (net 25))
 (segment (start 151.110001 155.250001) (end 151.86 156) (width 0.5) (layer B.Cu) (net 25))
 (segment (start 128.905 169.799) (end 138.061 169.799) (width 0.5) (layer B.Cu) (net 25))
 (segment (start 138.061 169.799) (end 151.86 156) (width 0.5) (layer B.Cu) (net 25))
 (segment (start 132.1 169.82) (end 128.926 169.82) (width 0.5) (layer F.Cu) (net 25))
 (segment (start 128.926 169.82) (end 128.905 169.799) (width 0.5) (layer F.Cu) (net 25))
 (via (at 128.905 169.799) (size 1.3) (drill 0.5) (layers F.Cu B.Cu) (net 25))
 (segment (start 109.855 181.345) (end 109.855 180.155) (width 0.5) (layer F.Cu) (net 7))
 (segment (start 109.855 180.155) (end 109.7 180) (width 0.5) (layer F.Cu) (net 7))
 (segment (start 121.559 168.55) (end 113.517 168.55) (width 0.5) (layer F.Cu) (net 7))
 (segment (start 109.7 172.367) (end 109.7 180) (width 0.5) (layer F.Cu) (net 7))
 (segment (start 113.517 168.55) (end 109.7 172.367) (width 0.5) (layer F.Cu) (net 7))
 (segment (start 121.559 164.74) (end 104.542 164.74) (width 0.5) (layer F.Cu) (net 13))
 (segment (start 104.542 164.74) (end 102.08 162.278) (width 0.5) (layer F.Cu) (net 13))
 (segment (start 102.08 162.278) (end 102.08 156) (width 0.5) (layer F.Cu) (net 13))
 (segment (start 107.350001 166.899999) (end 108 166.25) (width 0.5) (layer F.Cu) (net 28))
 (segment (start 99.748 167.132) (end 107.118 167.132) (width 0.5) (layer F.Cu) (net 28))
 (segment (start 107.118 167.132) (end 107.350001 166.899999) (width 0.5) (layer F.Cu) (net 28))
 (segment (start 108.649999 166.899999) (end 108 166.25) (width 0.5) (layer B.Cu) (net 28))
 (segment (start 110.279 168.529) (end 108.649999 166.899999) (width 0.5) (layer B.Cu) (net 28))
 (segment (start 123.444 168.529) (end 110.279 168.529) (width 0.5) (layer B.Cu) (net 28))
 (via (at 108 166.25) (size 1.3) (drill 0.5) (layers F.Cu B.Cu) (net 28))
 (segment (start 121.559 172.36) (end 122.694 172.36) (width 0.5) (layer F.Cu) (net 28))
 (segment (start 122.694 172.36) (end 123.444 171.61) (width 0.5) (layer F.Cu) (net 28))
 (segment (start 123.444 171.61) (end 123.444 168.529) (width 0.5) (layer F.Cu) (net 28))
 (via (at 123.444 168.529) (size 1.3) (drill 0.5) (layers F.Cu B.Cu) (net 28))
 (segment (start 105.250001 169.149999) (end 105.9 168.5) (width 0.5) (layer F.Cu) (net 29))
 (segment (start 104.728 169.672) (end 105.250001 169.149999) (width 0.5) (layer F.Cu) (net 29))
 (segment (start 106.549999 169.149999) (end 105.9 168.5) (width 0.5) (layer B.Cu) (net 29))
 (segment (start 107.199 169.799) (end 106.549999 169.149999) (width 0.5) (layer B.Cu) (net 29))
 (segment (start 99.748 169.672) (end 104.728 169.672) (width 0.5) (layer F.Cu) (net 29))
 (segment (start 124.968 169.799) (end 107.199 169.799) (width 0.5) (layer B.Cu) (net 29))
 (via (at 105.9 168.5) (size 1.3) (drill 0.5) (layers F.Cu B.Cu) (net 29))
 (segment (start 121.559 173.63) (end 123.169 173.63) (width 0.5) (layer F.Cu) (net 29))
 (via (at 124.968 169.799) (size 1.3) (drill 0.5) (layers F.Cu B.Cu) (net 29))
 (segment (start 124.968 171.831) (end 124.968 169.799) (width 0.5) (layer F.Cu) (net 29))
 (segment (start 123.169 173.63) (end 124.968 171.831) (width 0.5) (layer F.Cu) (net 29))
 (segment (start 100.002 169.418) (end 99.748 169.672) (width 0.5) (layer F.Cu) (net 29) (status 30))
 (segment (start 123.473998 154.5) (end 145.28 154.5) (width 0.5) (layer F.Cu) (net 10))
 (segment (start 145.28 154.5) (end 146.78 156) (width 0.5) (layer F.Cu) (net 10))
 (segment (start 120.1 160.2) (end 120.1 157.873998) (width 0.5) (layer F.Cu) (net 10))
 (segment (start 120.1 157.873998) (end 123.473998 154.5) (width 0.5) (layer F.Cu) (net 10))
 (segment (start 120.83 160.93) (end 120.1 160.2) (width 0.5) (layer F.Cu) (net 10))
 (segment (start 121.559 160.93) (end 120.83 160.93) (width 0.5) (layer F.Cu) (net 10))
 (segment (start 140.29 158.39) (end 151.86 169.96) (width 0.5) (layer F.Cu) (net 14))
 (segment (start 151.86 169.96) (end 151.86 180) (width 0.5) (layer F.Cu) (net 14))
 (segment (start 132.1 158.39) (end 140.29 158.39) (width 0.5) (layer F.Cu) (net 14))
 (segment (start 121.559 159.66) (end 122.694 159.66) (width 0.5) (layer F.Cu) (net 9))
 (segment (start 122.694 159.66) (end 124.954 157.4) (width 0.5) (layer F.Cu) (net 9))
 (segment (start 124.954 157.4) (end 140.3 157.4) (width 0.5) (layer F.Cu) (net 9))
 (segment (start 140.3 157.4) (end 140.950001 156.749999) (width 0.5) (layer F.Cu) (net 9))
 (segment (start 140.950001 156.749999) (end 141.7 156) (width 0.5) (layer F.Cu) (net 9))
 (segment (start 132.1 159.66) (end 139.06 159.66) (width 0.5) (layer F.Cu) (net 15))
 (segment (start 139.06 159.66) (end 149.32 169.92) (width 0.5) (layer F.Cu) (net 15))
 (segment (start 149.32 169.92) (end 149.32 180) (width 0.5) (layer F.Cu) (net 15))
 (segment (start 132.1 162.2) (end 134.7 162.2) (width 0.5) (layer F.Cu) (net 17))
 (segment (start 134.7 162.2) (end 136.62 164.12) (width 0.5) (layer F.Cu) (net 17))
 (segment (start 136.62 164.12) (end 136.62 180) (width 0.5) (layer F.Cu) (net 17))
 (segment (start 132.1 163.47) (end 133.235 163.47) (width 0.5) (layer F.Cu) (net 18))
 (segment (start 133.235 163.47) (end 134.08 164.315) (width 0.5) (layer F.Cu) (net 18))
 (segment (start 134.08 164.315) (end 134.08 178.93934) (width 0.5) (layer F.Cu) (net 18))
 (segment (start 134.08 178.93934) (end 134.08 180) (width 0.5) (layer F.Cu) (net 18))
 (segment (start 122.49 158.39) (end 124.88 156) (width 0.5) (layer F.Cu) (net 8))
 (segment (start 124.88 156) (end 134.08 156) (width 0.5) (layer F.Cu) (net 8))
 (segment (start 121.559 158.39) (end 122.49 158.39) (width 0.5) (layer F.Cu) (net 8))
 (segment (start 137.73 160.93) (end 141.7 164.9) (width 0.5) (layer F.Cu) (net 16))
 (segment (start 141.7 164.9) (end 141.7 180) (width 0.5) (layer F.Cu) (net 16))
 (segment (start 132.1 160.93) (end 137.73 160.93) (width 0.5) (layer F.Cu) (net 16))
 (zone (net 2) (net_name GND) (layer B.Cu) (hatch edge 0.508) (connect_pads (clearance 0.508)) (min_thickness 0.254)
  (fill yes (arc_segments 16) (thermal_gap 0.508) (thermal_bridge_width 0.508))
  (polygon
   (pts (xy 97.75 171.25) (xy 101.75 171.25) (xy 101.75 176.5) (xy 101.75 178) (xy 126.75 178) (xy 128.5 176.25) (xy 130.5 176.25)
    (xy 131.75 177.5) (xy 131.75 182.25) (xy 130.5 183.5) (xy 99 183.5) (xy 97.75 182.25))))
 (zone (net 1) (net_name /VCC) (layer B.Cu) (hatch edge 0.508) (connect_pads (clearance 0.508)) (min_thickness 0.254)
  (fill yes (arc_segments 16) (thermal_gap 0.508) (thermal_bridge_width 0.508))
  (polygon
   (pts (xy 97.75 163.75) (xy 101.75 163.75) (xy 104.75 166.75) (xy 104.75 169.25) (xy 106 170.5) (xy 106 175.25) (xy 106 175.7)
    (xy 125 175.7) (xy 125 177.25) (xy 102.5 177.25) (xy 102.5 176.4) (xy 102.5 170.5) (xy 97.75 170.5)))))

